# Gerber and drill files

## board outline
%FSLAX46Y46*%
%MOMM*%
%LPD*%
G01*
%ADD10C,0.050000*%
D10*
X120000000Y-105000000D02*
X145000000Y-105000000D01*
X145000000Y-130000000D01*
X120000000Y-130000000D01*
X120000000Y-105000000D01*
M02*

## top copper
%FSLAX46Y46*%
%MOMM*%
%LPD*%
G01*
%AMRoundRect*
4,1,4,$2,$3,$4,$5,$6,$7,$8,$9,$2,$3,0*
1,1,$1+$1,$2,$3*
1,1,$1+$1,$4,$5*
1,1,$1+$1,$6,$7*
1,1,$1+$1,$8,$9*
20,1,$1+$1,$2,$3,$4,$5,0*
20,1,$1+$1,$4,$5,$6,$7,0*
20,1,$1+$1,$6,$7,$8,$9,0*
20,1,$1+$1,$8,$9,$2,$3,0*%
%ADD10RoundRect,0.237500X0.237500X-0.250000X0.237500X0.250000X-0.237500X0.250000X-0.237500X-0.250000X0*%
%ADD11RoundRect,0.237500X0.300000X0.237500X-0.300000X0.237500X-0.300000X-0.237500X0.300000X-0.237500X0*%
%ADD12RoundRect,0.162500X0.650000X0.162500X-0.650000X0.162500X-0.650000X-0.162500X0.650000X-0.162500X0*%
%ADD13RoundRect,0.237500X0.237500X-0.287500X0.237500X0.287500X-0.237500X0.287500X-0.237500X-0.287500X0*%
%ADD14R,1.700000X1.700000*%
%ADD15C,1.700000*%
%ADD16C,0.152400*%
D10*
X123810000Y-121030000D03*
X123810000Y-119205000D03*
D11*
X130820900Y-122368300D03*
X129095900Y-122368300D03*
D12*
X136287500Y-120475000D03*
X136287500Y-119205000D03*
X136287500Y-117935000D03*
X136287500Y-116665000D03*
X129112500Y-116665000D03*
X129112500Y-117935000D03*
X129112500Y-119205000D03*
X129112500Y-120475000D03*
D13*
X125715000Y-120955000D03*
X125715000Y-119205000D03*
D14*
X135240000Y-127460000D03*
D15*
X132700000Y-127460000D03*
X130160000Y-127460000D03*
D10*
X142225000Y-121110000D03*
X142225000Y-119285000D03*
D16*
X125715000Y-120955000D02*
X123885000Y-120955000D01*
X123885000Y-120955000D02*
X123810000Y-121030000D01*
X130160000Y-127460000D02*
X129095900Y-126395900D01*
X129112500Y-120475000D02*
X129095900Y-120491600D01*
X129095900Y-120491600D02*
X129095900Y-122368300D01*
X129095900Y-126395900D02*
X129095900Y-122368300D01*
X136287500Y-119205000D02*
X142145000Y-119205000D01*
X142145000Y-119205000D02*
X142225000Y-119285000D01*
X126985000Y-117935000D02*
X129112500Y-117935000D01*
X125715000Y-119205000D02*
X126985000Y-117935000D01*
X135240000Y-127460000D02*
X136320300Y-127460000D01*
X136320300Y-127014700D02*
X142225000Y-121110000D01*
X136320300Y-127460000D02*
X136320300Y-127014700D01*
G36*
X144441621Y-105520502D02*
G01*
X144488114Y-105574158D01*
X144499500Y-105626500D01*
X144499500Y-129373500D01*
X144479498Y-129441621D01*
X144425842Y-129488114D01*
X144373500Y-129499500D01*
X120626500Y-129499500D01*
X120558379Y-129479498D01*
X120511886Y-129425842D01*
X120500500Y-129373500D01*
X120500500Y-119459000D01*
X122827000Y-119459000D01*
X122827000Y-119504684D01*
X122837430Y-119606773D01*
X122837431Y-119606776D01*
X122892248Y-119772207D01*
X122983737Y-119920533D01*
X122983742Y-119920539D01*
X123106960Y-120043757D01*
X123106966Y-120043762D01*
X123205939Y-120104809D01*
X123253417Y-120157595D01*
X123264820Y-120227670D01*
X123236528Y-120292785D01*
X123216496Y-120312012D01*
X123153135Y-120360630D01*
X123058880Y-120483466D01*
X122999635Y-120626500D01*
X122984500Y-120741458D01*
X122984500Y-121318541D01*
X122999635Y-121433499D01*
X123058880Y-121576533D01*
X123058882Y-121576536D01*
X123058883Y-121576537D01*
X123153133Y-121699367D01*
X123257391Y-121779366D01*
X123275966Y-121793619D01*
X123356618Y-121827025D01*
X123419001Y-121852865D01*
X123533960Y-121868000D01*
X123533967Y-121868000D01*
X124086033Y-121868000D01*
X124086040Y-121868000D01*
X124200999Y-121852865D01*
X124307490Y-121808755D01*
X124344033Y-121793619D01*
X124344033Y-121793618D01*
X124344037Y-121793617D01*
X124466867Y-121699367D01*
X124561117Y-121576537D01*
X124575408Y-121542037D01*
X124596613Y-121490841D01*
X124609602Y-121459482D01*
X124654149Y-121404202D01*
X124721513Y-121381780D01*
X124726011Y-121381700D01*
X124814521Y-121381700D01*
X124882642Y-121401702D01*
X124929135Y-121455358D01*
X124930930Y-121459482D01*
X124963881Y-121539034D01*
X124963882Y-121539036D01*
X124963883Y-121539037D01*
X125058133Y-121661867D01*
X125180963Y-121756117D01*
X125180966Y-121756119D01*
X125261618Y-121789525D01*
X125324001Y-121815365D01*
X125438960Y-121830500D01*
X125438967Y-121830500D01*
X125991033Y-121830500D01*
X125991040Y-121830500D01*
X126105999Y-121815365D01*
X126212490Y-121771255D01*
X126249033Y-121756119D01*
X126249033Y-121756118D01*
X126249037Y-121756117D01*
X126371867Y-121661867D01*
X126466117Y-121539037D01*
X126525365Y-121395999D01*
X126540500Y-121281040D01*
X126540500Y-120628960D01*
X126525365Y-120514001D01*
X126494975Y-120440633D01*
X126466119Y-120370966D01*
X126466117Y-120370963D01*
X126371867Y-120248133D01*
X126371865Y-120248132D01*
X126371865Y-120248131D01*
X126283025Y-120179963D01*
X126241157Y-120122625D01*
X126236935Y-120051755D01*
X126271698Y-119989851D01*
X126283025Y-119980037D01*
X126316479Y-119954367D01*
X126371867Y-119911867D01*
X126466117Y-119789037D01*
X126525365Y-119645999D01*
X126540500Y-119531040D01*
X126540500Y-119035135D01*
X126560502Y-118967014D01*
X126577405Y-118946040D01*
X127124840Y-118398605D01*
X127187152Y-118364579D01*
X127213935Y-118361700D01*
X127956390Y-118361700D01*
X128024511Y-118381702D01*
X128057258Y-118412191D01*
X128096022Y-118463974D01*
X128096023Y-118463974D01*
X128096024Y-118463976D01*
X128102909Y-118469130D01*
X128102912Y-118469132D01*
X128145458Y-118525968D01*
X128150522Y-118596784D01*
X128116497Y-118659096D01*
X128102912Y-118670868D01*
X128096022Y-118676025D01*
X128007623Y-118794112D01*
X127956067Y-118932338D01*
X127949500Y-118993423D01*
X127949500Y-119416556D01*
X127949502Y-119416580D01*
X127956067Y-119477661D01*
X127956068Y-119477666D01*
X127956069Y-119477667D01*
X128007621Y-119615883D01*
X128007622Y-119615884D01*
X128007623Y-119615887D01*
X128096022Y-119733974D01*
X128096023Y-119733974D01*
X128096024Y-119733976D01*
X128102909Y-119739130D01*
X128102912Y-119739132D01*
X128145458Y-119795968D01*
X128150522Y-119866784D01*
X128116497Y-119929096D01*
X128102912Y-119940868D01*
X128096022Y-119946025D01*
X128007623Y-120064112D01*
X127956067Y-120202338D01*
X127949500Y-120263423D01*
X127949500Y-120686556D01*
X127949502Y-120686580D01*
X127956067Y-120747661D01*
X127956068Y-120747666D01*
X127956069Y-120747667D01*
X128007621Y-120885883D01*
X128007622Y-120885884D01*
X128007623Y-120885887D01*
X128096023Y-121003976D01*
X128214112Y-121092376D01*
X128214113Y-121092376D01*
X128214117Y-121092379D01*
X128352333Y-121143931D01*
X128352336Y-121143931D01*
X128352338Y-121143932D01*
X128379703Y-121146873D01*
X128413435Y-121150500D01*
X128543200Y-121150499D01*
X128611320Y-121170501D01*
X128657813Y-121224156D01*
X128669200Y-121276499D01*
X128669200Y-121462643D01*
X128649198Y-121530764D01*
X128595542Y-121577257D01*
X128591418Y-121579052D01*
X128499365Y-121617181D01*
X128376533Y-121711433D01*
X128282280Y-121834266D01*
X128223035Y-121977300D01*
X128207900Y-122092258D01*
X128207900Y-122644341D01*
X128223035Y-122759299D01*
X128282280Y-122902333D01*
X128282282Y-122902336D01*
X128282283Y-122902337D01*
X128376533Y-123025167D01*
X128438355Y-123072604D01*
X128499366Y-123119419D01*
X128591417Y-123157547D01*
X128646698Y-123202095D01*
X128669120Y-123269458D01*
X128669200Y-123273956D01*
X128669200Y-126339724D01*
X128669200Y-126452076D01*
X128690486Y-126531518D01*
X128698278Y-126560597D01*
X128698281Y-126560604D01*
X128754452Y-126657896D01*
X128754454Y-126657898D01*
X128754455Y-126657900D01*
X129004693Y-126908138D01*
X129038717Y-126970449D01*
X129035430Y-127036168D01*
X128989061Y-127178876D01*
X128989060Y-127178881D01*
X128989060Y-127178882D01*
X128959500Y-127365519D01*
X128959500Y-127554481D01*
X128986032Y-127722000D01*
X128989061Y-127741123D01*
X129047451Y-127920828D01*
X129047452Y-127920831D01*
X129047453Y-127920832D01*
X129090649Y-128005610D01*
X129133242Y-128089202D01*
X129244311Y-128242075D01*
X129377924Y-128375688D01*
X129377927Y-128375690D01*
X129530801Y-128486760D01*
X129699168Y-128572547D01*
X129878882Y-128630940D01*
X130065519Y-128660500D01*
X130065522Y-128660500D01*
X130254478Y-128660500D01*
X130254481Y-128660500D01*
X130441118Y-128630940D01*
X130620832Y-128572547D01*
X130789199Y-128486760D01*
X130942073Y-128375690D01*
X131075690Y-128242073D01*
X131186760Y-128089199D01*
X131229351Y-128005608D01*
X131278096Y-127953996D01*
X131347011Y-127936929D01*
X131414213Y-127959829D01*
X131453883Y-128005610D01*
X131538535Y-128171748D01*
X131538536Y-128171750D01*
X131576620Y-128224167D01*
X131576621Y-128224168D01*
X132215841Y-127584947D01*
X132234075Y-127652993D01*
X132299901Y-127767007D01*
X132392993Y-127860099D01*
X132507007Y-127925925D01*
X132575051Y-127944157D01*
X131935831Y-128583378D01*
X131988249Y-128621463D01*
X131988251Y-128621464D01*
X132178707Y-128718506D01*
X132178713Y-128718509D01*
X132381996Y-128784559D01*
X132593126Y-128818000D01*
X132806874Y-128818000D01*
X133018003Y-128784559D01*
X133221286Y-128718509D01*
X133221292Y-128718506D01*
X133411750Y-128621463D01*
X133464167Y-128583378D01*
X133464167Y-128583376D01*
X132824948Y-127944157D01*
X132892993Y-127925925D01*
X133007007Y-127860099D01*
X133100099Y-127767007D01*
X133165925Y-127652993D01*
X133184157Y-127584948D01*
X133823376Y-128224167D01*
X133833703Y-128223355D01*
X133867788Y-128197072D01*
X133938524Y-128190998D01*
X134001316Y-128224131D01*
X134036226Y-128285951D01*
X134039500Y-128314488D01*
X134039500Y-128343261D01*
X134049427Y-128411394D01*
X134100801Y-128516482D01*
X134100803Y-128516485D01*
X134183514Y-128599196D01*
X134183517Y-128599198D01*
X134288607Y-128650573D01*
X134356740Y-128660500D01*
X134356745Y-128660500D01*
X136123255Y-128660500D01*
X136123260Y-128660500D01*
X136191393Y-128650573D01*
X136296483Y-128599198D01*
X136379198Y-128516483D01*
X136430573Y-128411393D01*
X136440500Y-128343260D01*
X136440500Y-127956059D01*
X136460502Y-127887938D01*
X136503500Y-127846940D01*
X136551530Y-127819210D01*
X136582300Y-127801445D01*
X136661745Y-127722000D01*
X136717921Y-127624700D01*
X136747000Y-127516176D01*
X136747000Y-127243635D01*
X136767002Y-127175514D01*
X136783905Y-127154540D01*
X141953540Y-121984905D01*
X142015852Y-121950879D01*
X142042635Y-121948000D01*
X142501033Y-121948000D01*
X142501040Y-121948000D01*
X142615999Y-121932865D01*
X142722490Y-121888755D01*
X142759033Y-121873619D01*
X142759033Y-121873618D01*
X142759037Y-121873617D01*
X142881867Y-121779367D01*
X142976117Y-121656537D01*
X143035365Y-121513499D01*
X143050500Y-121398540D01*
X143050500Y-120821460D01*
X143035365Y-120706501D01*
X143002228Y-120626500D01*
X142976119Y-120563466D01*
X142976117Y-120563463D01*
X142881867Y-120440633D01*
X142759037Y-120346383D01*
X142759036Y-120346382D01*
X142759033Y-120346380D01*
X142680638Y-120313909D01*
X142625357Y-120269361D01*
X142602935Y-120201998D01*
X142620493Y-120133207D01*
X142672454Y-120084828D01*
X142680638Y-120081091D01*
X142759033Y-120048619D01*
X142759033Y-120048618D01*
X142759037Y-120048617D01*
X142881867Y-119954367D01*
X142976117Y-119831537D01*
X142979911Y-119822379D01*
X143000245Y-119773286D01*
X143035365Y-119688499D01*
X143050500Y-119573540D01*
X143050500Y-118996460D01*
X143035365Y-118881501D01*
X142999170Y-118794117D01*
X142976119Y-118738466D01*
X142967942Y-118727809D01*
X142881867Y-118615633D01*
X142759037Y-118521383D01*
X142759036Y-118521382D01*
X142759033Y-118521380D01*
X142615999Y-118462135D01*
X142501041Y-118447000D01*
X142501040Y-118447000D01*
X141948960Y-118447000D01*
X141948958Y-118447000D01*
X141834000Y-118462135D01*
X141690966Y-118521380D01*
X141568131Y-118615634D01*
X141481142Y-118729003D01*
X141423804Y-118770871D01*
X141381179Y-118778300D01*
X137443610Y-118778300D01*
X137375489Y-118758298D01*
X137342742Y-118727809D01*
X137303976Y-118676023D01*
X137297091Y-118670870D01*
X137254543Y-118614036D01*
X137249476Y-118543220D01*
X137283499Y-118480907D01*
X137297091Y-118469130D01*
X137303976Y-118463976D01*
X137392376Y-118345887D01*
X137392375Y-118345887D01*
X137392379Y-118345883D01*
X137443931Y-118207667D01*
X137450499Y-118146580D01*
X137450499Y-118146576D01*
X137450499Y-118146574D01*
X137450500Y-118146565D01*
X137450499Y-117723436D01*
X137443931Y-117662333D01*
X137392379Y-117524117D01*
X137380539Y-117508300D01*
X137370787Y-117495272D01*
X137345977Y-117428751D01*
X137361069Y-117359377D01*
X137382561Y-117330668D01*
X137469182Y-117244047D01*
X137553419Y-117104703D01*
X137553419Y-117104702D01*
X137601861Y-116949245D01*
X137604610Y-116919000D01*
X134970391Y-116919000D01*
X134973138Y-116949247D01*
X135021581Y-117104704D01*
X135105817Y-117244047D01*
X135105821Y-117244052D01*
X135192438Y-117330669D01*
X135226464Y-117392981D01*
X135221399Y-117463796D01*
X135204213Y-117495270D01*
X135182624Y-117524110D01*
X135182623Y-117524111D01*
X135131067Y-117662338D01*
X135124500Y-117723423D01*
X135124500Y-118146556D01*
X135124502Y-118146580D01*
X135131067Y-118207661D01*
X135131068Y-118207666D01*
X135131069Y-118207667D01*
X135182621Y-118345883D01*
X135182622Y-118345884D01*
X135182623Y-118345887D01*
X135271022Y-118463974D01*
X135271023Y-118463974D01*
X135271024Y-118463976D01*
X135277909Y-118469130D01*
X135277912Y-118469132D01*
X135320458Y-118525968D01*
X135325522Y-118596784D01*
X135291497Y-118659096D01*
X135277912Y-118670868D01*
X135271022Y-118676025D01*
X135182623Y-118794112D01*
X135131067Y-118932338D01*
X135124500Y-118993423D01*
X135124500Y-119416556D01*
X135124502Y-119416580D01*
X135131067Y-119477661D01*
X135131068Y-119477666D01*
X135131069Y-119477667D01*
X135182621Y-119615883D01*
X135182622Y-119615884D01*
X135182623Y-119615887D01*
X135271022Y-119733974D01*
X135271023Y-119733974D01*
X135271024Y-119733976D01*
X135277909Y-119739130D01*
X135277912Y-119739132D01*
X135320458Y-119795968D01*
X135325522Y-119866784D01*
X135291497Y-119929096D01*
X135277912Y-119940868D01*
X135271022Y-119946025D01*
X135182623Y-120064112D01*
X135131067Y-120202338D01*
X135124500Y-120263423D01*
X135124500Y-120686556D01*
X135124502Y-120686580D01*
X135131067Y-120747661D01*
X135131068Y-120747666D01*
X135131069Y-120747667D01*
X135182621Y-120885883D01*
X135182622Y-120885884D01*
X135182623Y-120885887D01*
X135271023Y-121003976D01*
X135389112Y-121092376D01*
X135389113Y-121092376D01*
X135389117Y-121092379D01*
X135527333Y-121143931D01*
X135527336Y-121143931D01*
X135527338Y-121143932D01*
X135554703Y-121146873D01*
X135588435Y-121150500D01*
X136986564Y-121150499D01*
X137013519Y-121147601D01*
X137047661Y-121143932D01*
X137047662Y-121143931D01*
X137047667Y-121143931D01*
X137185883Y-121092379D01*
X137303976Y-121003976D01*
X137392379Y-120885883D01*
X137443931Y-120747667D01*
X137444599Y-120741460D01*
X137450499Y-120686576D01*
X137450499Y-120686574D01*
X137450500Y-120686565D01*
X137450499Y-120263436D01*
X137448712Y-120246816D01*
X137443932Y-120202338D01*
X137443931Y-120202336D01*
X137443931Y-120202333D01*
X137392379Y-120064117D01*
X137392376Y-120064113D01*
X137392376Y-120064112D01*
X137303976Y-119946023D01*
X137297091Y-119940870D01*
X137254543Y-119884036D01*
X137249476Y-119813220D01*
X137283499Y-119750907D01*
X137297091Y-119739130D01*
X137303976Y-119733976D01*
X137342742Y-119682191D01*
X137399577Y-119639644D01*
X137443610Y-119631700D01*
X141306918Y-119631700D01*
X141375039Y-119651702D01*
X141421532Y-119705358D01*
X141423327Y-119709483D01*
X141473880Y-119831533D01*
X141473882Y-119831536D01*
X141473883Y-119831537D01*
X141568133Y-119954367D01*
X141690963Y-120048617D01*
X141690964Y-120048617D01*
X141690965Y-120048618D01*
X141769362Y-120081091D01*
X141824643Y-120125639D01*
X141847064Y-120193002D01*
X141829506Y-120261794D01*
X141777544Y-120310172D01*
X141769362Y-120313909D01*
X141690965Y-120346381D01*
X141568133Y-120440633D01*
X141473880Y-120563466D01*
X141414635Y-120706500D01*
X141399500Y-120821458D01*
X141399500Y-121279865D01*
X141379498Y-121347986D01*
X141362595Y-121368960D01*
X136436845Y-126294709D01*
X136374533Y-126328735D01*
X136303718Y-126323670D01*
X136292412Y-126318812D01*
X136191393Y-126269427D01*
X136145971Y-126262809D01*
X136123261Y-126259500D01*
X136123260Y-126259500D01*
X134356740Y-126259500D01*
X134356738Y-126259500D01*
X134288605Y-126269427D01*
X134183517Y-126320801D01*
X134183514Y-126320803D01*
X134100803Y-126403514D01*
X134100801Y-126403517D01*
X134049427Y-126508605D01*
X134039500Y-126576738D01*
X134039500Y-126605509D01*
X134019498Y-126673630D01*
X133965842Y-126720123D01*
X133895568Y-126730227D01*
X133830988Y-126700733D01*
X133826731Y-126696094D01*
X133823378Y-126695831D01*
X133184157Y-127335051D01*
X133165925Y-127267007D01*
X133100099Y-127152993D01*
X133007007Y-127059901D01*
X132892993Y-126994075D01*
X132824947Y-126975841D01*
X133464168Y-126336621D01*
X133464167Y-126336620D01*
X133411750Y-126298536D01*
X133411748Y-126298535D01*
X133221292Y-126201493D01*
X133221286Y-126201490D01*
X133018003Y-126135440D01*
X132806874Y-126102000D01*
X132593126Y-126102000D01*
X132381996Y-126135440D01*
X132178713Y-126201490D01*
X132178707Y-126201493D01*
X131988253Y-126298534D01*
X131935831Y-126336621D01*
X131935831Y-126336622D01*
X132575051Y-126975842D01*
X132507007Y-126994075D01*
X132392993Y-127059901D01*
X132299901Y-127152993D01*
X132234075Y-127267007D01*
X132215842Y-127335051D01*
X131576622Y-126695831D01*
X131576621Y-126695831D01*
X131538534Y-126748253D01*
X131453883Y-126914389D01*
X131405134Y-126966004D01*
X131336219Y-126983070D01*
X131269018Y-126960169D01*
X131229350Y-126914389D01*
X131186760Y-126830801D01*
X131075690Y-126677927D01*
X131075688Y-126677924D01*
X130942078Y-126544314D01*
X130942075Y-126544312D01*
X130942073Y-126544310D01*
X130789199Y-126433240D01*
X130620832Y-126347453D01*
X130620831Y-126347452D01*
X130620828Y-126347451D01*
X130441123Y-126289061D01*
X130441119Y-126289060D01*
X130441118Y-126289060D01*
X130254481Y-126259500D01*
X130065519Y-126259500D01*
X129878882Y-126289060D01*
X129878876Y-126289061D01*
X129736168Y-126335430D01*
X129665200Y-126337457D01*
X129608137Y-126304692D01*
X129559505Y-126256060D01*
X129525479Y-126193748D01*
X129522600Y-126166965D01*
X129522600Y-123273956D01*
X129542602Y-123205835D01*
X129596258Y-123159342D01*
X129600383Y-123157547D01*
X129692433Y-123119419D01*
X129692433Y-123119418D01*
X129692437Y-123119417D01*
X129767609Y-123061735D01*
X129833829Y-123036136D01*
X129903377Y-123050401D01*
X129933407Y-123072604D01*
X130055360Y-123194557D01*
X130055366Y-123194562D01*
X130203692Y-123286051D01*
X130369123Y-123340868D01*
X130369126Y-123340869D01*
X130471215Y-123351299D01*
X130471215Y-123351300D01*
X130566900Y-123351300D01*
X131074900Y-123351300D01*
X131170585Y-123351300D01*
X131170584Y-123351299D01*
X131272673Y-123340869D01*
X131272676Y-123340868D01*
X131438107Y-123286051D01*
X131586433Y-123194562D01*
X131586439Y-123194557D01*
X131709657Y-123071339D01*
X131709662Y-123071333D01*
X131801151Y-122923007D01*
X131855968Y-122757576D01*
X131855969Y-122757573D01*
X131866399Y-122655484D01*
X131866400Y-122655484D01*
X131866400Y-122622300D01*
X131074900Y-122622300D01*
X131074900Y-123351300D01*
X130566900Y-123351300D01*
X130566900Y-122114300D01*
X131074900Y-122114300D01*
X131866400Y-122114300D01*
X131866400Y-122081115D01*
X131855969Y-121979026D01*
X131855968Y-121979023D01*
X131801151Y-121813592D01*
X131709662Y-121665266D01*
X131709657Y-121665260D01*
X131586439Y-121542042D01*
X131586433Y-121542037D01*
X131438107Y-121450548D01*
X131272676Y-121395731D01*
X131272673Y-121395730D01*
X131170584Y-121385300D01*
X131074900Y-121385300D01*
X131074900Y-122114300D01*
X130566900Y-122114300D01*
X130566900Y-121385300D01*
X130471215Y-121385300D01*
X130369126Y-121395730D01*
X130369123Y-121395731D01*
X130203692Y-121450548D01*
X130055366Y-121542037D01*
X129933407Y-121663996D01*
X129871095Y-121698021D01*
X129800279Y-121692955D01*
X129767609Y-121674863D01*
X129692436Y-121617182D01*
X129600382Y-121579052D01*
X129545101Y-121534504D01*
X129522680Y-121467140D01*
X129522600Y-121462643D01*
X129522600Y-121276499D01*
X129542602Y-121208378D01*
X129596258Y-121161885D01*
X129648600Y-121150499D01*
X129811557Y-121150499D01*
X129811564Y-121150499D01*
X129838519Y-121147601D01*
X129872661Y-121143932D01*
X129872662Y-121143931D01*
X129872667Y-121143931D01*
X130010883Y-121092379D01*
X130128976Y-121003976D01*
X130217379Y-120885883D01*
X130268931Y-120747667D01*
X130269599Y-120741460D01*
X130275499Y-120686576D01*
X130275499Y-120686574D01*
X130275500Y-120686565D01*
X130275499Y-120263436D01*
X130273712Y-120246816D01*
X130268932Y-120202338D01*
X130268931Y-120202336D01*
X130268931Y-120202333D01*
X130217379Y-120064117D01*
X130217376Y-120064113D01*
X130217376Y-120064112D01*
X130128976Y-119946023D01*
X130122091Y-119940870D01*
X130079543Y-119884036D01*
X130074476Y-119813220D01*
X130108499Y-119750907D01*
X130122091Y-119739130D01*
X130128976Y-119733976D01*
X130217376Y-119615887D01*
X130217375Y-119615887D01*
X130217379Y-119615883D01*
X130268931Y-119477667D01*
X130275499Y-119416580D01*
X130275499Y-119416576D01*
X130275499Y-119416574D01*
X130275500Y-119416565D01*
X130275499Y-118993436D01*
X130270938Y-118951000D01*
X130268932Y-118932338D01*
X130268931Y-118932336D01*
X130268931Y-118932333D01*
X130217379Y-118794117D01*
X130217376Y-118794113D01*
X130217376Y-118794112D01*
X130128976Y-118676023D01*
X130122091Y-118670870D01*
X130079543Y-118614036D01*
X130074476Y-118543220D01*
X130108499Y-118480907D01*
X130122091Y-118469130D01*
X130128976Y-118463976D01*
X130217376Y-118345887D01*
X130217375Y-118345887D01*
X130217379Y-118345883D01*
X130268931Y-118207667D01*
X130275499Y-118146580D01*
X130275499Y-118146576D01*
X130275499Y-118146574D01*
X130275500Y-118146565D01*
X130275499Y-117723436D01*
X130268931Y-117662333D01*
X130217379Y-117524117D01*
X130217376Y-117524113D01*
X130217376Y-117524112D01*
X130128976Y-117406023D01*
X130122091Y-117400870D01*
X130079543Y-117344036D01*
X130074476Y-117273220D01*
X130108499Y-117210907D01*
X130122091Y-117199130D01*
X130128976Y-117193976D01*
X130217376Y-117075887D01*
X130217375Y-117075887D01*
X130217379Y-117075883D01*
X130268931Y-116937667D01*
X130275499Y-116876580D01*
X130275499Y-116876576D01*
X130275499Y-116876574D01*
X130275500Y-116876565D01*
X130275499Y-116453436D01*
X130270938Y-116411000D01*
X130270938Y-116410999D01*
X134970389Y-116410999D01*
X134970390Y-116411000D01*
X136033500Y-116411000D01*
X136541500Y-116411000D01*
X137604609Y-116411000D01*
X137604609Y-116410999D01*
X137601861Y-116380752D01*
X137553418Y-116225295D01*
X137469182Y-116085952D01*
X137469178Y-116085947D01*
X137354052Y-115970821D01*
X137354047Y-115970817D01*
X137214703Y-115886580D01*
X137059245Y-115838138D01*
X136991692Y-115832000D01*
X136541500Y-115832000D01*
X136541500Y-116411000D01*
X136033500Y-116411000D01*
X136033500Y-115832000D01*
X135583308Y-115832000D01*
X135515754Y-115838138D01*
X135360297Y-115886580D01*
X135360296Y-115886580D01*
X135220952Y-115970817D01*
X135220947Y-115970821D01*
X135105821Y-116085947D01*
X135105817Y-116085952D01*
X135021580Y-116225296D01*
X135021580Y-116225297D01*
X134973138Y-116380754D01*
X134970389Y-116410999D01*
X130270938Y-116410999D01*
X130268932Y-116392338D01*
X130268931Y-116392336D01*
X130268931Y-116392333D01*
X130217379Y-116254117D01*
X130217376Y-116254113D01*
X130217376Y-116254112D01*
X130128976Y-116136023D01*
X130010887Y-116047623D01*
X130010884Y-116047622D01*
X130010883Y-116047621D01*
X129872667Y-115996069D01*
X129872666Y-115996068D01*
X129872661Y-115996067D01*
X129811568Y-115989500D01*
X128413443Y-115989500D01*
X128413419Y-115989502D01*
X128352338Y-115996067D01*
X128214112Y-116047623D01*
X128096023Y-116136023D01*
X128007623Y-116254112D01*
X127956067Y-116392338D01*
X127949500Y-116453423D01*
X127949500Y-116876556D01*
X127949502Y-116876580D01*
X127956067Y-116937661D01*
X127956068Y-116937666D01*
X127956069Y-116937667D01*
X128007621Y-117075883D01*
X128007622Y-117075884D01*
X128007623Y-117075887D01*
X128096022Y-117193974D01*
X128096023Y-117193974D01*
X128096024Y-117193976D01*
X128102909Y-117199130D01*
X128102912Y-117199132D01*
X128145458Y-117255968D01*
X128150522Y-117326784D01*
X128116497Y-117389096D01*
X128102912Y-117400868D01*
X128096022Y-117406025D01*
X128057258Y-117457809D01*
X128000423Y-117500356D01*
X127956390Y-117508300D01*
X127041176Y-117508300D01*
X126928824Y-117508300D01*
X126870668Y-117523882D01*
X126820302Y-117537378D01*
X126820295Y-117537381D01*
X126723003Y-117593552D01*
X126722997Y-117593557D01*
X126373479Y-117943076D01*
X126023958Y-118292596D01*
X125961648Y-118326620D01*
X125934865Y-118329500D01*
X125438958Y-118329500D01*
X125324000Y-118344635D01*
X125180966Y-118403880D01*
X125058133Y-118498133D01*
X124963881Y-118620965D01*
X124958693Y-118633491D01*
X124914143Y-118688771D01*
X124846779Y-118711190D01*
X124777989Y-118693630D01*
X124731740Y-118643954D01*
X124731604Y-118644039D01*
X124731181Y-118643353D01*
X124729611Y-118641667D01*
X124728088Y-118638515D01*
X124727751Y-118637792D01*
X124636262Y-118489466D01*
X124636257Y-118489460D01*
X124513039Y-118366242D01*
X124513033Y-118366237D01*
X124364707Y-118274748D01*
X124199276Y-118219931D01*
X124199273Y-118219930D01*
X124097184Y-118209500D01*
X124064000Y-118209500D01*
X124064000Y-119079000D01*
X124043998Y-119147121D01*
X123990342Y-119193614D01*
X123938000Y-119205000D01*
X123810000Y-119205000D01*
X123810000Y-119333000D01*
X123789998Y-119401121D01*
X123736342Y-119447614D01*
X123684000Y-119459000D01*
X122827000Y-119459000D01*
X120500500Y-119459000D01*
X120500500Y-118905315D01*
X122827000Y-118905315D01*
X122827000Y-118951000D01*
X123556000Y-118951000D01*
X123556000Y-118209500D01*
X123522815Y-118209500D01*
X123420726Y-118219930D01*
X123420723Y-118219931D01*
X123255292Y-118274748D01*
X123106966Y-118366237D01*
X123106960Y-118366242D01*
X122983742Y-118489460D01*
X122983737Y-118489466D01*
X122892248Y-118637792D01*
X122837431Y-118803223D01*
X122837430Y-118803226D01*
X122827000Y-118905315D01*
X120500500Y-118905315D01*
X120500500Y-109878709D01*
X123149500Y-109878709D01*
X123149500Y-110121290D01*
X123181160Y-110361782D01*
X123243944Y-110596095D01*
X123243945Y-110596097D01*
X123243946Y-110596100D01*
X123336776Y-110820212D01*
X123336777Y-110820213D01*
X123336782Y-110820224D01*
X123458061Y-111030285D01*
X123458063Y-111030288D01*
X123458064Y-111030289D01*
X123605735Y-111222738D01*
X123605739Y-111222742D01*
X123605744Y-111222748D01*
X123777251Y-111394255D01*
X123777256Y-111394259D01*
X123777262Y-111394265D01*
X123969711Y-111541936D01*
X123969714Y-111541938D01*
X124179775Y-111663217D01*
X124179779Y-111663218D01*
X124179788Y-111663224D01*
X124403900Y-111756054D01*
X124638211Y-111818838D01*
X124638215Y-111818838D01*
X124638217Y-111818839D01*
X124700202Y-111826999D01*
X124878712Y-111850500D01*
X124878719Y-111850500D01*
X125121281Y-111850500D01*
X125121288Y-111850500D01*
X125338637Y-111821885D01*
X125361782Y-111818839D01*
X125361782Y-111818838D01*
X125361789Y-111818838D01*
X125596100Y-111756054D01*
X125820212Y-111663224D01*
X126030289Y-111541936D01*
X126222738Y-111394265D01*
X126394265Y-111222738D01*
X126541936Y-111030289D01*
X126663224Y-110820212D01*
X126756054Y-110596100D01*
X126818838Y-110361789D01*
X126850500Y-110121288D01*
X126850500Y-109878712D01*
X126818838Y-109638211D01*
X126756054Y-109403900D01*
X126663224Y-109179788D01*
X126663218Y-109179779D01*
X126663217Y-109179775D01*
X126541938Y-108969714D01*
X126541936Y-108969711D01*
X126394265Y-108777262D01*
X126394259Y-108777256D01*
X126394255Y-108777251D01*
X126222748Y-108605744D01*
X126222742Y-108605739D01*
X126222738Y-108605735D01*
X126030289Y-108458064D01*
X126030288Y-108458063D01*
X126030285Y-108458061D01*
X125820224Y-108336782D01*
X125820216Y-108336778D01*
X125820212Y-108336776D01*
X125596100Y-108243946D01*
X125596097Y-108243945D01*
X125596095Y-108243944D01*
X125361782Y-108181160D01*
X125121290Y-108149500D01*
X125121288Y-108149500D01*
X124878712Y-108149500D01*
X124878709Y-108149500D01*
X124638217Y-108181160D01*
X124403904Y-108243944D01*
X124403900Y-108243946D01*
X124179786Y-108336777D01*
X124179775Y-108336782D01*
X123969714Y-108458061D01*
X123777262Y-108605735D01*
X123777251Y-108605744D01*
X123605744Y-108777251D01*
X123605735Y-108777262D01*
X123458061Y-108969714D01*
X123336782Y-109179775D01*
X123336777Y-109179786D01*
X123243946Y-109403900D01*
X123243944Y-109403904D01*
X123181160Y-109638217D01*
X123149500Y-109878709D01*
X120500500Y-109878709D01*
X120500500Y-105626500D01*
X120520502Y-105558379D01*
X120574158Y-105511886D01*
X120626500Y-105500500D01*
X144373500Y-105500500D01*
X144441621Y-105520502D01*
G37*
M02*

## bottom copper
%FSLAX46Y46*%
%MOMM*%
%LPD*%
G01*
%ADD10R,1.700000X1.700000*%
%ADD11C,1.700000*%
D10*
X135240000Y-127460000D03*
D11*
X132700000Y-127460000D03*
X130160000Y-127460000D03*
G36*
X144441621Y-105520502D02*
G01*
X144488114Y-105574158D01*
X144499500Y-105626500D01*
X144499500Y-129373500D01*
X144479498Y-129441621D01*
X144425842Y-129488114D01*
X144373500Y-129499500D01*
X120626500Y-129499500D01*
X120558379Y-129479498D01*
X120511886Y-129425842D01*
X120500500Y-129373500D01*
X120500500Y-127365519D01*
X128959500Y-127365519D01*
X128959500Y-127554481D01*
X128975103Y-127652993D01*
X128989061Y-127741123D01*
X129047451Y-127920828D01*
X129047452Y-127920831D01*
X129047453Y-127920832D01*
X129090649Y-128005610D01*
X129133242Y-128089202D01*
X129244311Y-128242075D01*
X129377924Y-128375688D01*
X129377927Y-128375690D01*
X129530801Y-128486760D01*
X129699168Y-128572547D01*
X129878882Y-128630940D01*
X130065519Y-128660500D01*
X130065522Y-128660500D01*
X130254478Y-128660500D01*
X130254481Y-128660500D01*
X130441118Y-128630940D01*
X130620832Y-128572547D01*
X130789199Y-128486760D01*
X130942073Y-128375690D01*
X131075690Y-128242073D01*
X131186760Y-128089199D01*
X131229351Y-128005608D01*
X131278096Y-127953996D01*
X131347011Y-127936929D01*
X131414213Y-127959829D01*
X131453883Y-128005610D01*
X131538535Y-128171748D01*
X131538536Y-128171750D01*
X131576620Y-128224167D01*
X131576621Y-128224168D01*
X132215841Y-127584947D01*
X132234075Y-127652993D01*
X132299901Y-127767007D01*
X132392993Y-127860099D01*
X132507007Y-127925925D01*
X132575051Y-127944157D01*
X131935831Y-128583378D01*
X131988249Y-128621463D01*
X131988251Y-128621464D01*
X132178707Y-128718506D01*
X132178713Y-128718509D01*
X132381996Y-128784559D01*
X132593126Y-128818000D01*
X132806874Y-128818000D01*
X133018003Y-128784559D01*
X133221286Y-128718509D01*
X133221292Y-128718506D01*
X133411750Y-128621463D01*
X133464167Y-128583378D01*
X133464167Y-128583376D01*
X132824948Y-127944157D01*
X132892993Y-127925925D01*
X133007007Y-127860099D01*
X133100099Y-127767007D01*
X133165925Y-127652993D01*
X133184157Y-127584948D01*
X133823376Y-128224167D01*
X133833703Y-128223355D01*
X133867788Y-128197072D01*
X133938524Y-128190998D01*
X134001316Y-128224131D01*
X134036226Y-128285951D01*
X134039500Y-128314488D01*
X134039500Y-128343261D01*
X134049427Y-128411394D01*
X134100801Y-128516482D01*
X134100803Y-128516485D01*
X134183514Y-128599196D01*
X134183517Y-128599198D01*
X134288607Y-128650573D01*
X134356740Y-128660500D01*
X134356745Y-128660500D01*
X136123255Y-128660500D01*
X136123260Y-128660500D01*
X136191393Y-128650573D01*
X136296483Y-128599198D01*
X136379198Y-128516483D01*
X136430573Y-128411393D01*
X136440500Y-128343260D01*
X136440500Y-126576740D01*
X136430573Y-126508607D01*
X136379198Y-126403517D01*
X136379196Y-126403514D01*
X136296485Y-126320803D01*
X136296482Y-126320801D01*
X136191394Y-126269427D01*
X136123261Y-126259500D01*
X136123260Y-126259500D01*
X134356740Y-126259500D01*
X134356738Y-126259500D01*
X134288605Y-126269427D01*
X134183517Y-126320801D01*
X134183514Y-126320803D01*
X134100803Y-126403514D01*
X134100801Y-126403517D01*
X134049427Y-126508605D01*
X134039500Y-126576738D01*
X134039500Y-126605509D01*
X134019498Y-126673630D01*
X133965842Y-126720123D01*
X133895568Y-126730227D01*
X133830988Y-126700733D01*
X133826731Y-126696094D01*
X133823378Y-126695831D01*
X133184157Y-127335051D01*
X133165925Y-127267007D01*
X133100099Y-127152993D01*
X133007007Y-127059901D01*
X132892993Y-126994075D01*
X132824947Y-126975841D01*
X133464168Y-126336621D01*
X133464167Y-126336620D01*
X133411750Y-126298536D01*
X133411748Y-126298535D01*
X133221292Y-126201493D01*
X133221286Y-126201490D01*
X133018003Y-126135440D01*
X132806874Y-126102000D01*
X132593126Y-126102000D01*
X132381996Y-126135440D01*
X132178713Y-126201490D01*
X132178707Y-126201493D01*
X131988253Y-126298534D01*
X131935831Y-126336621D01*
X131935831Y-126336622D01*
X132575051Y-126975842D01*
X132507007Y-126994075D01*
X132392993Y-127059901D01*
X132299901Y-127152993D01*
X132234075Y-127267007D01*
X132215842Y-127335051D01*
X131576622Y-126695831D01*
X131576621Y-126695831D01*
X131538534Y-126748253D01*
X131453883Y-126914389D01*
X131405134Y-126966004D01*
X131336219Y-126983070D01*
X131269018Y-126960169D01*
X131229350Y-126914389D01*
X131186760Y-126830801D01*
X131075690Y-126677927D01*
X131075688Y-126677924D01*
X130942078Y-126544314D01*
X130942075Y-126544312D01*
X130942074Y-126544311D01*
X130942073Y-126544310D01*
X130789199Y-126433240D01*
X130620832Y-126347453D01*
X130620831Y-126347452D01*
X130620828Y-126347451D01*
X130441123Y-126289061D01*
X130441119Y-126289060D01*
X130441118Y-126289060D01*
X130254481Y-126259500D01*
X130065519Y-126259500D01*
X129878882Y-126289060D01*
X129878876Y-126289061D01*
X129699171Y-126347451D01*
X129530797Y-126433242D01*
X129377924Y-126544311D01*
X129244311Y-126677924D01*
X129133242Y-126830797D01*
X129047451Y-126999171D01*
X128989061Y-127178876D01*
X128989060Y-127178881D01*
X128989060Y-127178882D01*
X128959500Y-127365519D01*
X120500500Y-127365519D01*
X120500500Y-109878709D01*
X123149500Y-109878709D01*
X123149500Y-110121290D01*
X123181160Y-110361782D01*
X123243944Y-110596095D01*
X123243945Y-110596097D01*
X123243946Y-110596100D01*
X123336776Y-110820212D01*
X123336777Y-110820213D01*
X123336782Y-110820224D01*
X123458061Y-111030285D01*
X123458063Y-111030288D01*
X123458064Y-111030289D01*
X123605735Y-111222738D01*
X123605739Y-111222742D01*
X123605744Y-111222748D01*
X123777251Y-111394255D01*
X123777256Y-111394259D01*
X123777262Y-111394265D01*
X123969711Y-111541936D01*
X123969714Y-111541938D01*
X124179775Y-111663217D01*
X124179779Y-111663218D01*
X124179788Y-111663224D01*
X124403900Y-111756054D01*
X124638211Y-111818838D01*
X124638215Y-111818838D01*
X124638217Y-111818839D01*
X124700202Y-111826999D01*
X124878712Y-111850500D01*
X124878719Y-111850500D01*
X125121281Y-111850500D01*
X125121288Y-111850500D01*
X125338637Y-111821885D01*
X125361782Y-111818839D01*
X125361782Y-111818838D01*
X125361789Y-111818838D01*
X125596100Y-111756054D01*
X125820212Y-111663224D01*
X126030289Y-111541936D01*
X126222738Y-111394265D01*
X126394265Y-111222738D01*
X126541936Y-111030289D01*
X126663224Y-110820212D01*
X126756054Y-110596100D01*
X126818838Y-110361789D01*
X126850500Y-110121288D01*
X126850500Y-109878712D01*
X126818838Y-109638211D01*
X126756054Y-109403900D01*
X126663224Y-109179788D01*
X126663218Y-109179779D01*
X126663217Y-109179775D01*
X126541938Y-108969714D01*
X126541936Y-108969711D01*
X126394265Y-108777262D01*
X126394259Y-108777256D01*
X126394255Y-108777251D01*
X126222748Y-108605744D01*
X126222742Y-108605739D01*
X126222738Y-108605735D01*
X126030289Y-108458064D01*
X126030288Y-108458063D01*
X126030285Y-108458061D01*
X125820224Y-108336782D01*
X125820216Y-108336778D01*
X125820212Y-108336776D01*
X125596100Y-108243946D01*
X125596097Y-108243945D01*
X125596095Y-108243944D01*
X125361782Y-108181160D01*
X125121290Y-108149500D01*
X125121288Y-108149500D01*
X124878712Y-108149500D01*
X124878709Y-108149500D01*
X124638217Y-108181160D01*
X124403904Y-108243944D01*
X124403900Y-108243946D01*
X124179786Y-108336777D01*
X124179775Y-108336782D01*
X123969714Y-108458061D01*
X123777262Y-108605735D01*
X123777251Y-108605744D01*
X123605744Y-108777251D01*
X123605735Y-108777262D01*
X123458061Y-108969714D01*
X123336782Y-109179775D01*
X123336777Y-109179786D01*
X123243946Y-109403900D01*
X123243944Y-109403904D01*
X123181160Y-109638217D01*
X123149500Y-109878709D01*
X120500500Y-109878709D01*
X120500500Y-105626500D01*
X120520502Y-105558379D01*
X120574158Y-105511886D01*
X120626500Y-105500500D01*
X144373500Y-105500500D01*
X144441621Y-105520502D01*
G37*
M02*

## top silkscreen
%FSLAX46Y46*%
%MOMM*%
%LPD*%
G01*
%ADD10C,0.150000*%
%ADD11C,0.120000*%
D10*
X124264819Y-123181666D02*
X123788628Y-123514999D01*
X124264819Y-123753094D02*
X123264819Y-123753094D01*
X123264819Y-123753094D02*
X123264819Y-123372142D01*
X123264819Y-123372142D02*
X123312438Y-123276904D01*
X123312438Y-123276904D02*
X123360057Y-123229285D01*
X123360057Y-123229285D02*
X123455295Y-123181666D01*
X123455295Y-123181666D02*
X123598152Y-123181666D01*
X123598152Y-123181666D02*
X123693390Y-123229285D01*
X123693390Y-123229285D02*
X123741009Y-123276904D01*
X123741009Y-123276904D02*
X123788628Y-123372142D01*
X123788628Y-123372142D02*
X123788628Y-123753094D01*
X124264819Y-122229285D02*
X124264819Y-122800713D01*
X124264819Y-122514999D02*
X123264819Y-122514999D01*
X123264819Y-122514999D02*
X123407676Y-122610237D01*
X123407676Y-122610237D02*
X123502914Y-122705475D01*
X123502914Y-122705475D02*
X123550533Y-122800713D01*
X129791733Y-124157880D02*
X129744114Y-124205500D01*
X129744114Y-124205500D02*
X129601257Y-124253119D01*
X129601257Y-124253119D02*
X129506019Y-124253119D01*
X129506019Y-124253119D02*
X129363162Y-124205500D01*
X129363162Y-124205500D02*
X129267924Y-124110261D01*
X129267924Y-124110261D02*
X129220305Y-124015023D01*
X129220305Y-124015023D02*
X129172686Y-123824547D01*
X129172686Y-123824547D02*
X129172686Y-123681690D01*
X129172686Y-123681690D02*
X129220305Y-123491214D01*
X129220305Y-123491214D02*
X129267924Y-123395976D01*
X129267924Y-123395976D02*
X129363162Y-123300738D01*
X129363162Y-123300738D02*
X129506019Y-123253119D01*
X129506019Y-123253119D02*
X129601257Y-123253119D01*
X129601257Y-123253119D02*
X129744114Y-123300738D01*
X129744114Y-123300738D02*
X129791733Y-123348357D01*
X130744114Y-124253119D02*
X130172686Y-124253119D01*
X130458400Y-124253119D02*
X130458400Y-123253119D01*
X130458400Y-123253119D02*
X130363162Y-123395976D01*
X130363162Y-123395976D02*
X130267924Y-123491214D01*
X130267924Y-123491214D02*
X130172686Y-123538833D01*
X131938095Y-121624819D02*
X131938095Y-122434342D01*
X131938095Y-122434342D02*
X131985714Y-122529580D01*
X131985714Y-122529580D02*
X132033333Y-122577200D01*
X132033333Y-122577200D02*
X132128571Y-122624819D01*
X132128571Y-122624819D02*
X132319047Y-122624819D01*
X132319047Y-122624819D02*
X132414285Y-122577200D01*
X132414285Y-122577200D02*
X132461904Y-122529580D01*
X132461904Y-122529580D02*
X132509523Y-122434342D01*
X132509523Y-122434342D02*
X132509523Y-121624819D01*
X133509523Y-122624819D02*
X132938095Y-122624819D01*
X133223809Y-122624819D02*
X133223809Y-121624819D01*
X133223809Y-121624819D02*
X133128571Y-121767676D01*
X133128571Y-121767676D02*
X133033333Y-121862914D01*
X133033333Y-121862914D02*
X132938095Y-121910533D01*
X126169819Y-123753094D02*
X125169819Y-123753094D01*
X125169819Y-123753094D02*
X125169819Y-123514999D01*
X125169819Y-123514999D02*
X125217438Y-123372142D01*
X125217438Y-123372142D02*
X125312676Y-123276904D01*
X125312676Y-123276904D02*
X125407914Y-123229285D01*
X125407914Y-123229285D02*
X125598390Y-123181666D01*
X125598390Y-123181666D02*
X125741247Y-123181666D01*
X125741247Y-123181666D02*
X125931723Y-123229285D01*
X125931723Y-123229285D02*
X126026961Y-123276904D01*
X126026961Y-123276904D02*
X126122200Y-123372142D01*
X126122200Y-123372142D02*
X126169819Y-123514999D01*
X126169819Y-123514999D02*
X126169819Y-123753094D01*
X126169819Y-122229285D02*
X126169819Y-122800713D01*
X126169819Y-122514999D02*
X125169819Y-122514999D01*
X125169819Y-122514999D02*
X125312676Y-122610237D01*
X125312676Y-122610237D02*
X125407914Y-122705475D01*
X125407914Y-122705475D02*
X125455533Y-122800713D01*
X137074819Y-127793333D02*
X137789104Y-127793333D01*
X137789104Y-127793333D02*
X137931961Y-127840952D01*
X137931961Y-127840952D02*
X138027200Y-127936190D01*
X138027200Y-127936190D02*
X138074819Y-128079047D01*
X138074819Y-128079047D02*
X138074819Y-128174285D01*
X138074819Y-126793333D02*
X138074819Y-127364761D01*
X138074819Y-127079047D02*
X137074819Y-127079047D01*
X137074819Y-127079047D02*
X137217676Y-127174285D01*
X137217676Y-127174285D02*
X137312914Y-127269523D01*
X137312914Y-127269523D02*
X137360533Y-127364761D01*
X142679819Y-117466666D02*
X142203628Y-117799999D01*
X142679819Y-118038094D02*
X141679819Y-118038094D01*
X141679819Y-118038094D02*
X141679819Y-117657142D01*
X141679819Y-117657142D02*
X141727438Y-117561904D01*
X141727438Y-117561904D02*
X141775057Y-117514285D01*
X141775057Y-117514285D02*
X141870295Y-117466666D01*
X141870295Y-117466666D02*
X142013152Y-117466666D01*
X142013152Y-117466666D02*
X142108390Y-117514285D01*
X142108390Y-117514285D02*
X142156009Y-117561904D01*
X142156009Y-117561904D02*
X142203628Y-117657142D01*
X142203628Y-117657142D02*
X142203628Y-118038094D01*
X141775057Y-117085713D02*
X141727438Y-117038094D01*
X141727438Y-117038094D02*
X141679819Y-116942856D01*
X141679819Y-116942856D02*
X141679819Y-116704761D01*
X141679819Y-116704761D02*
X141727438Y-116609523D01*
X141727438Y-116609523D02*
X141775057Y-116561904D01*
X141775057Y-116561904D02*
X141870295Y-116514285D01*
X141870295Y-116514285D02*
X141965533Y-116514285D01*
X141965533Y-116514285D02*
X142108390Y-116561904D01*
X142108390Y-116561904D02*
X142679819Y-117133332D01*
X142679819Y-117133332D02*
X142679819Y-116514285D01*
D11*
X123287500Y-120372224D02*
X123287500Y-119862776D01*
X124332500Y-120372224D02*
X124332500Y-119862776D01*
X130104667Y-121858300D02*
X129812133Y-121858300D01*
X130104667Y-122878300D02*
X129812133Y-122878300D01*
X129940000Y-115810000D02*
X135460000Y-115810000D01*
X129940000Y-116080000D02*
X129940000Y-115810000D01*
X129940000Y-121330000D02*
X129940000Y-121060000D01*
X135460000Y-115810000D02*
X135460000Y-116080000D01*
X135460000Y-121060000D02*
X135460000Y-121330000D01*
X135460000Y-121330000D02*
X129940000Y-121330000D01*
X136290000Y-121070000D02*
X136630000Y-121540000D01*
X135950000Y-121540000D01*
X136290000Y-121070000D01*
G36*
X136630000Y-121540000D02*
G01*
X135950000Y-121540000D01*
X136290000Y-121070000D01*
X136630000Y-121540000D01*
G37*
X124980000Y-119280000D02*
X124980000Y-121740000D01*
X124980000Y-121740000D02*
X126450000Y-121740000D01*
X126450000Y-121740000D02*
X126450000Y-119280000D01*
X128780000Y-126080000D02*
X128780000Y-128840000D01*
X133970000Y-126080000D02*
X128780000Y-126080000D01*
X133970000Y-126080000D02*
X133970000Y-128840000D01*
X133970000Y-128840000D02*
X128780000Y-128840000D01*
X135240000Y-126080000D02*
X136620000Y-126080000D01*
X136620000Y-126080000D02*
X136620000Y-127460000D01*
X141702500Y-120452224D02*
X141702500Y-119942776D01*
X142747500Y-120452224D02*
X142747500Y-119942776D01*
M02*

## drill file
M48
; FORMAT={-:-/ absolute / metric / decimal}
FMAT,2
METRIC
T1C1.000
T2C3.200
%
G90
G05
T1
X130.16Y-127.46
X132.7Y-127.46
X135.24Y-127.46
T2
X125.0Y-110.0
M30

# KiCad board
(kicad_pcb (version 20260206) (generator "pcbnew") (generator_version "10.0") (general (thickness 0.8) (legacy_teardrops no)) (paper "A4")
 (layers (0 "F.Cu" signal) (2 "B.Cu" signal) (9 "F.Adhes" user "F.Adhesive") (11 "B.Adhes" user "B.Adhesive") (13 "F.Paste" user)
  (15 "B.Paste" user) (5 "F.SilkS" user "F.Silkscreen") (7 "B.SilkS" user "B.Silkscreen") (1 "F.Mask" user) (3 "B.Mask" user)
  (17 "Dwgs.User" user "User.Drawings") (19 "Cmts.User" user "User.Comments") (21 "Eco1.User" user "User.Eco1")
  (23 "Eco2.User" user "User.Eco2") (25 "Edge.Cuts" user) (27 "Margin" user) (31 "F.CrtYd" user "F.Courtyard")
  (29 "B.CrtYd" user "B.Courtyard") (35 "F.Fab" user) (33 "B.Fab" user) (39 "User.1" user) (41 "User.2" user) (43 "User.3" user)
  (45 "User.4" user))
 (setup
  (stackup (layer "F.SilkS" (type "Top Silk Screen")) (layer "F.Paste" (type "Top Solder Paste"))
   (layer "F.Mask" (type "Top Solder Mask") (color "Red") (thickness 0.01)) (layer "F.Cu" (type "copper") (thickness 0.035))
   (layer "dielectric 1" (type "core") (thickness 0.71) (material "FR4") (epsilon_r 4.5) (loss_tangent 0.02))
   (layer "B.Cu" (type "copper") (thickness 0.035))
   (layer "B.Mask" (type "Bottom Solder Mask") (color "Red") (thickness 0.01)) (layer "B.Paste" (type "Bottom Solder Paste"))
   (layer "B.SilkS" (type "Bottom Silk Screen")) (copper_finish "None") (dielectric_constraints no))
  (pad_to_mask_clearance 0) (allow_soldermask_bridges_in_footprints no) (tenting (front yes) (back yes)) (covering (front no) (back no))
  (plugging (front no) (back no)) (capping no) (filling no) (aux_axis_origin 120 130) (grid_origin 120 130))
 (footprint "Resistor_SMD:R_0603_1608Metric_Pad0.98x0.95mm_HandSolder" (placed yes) (layer "F.Cu") (at 123.81 120.1175 90)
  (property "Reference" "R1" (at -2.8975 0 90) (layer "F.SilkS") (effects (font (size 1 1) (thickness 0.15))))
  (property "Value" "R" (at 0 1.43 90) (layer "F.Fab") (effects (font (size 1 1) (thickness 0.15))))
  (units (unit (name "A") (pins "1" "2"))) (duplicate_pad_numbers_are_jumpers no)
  (fp_line (start -0.254724 -0.5225) (end 0.254724 -0.5225) (stroke (width 0.12) (type solid)) (layer "F.SilkS"))
  (fp_line (start -0.254724 0.5225) (end 0.254724 0.5225) (stroke (width 0.12) (type solid)) (layer "F.SilkS"))
  (pad "1" smd roundrect (at -0.9125 0 90) (size 0.975 0.95) (layers "F.Cu" "F.Mask" "F.Paste") (roundrect_rratio 0.25) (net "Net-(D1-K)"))
  (pad "2" smd roundrect (at 0.9125 0 90) (size 0.975 0.95) (layers "F.Cu" "F.Mask" "F.Paste") (roundrect_rratio 0.25) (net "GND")))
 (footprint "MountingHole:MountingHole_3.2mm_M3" (layer "F.Cu") (at 125 110)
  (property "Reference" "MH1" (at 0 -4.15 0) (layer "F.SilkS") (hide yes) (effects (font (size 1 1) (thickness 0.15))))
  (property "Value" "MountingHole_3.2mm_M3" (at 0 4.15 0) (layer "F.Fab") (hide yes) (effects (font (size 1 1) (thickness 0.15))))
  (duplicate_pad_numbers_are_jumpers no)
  (pad "" np_thru_hole circle (at 0 0) (size 3.2 3.2) (drill 3.2) (layers "*.Cu" "*.Mask")))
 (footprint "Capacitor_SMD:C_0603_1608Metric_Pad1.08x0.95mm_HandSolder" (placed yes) (layer "F.Cu") (at 129.9584 122.3683 180)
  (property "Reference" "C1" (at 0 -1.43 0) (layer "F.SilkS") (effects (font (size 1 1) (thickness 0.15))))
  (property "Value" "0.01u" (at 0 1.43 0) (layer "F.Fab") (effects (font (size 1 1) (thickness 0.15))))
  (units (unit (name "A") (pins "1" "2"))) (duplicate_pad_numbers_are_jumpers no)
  (fp_line (start -0.146267 0.51) (end 0.146267 0.51) (stroke (width 0.12) (type solid)) (layer "F.SilkS"))
  (fp_line (start -0.146267 -0.51) (end 0.146267 -0.51) (stroke (width 0.12) (type solid)) (layer "F.SilkS"))
  (pad "1" smd roundrect (at -0.8625 0 180) (size 1.075 0.95) (layers "F.Cu" "F.Mask" "F.Paste") (roundrect_rratio 0.25) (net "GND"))
  (pad "2" smd roundrect (at 0.8625 0 180) (size 1.075 0.95) (layers "F.Cu" "F.Mask" "F.Paste") (roundrect_rratio 0.25) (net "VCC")))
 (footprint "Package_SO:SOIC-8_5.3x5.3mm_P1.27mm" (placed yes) (layer "F.Cu") (at 132.7 118.57 180)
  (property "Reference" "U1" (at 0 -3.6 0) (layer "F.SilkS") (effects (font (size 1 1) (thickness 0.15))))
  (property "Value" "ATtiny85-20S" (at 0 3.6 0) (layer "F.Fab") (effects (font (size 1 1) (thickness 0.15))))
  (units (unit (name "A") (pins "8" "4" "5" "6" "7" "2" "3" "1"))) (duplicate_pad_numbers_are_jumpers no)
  (fp_line (start 2.76 2.76) (end -2.76 2.76) (stroke (width 0.12) (type solid)) (layer "F.SilkS"))
  (fp_line (start 2.76 2.49) (end 2.76 2.76) (stroke (width 0.12) (type solid)) (layer "F.SilkS"))
  (fp_line (start 2.76 -2.76) (end 2.76 -2.49) (stroke (width 0.12) (type solid)) (layer "F.SilkS"))
  (fp_line (start -2.76 2.76) (end -2.76 2.49) (stroke (width 0.12) (type solid)) (layer "F.SilkS"))
  (fp_line (start -2.76 -2.49) (end -2.76 -2.76) (stroke (width 0.12) (type solid)) (layer "F.SilkS"))
  (fp_line (start -2.76 -2.76) (end 2.76 -2.76) (stroke (width 0.12) (type solid)) (layer "F.SilkS"))
  (fp_poly (pts (xy -3.59 -2.5) (xy -3.93 -2.97) (xy -3.25 -2.97)) (stroke (width 0.12) (type solid)) (fill yes) (layer "F.SilkS"))
  (pad "1" smd roundrect (at -3.5875 -1.905 180) (size 1.625 0.65) (layers "F.Cu" "F.Mask" "F.Paste") (roundrect_rratio 0.25)
   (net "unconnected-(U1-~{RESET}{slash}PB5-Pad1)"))
  (pad "2" smd roundrect (at -3.5875 -0.635 180) (size 1.625 0.65) (layers "F.Cu" "F.Mask" "F.Paste") (roundrect_rratio 0.25) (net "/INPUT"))
  (pad "3" smd roundrect (at -3.5875 0.635 180) (size 1.625 0.65) (layers "F.Cu" "F.Mask" "F.Paste") (roundrect_rratio 0.25)
   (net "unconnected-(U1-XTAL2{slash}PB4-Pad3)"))
  (pad "4" smd roundrect (at -3.5875 1.905 180) (size 1.625 0.65) (layers "F.Cu" "F.Mask" "F.Paste") (roundrect_rratio 0.25) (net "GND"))
  (pad "5" smd roundrect (at 3.5875 1.905 180) (size 1.625 0.65) (layers "F.Cu" "F.Mask" "F.Paste") (roundrect_rratio 0.25)
   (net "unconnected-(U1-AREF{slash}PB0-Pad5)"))
  (pad "6" smd roundrect (at 3.5875 0.635 180) (size 1.625 0.65) (layers "F.Cu" "F.Mask" "F.Paste") (roundrect_rratio 0.25)
   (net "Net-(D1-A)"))
  (pad "7" smd roundrect (at 3.5875 -0.635 180) (size 1.625 0.65) (layers "F.Cu" "F.Mask" "F.Paste") (roundrect_rratio 0.25)
   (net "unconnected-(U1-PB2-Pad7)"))
  (pad "8" smd roundrect (at 3.5875 -1.905 180) (size 1.625 0.65) (layers "F.Cu" "F.Mask" "F.Paste") (roundrect_rratio 0.25) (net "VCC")))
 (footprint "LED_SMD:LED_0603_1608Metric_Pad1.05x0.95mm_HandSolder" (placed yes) (layer "F.Cu") (at 125.715 120.08 90)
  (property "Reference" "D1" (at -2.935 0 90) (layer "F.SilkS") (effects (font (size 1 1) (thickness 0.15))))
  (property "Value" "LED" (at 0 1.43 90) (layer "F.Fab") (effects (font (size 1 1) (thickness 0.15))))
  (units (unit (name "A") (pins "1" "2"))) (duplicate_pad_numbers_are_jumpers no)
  (fp_line (start 0.8 -0.735) (end -1.66 -0.735) (stroke (width 0.12) (type solid)) (layer "F.SilkS"))
  (fp_line (start -1.66 -0.735) (end -1.66 0.735) (stroke (width 0.12) (type solid)) (layer "F.SilkS"))
  (fp_line (start -1.66 0.735) (end 0.8 0.735) (stroke (width 0.12) (type solid)) (layer "F.SilkS"))
  (pad "1" smd roundrect (at -0.875 0 90) (size 1.05 0.95) (layers "F.Cu" "F.Mask" "F.Paste") (roundrect_rratio 0.25) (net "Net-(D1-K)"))
  (pad "2" smd roundrect (at 0.875 0 90) (size 1.05 0.95) (layers "F.Cu" "F.Mask" "F.Paste") (roundrect_rratio 0.25) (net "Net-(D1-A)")))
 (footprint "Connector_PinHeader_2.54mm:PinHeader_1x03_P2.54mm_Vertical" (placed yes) (layer "F.Cu") (at 135.24 127.46 -90)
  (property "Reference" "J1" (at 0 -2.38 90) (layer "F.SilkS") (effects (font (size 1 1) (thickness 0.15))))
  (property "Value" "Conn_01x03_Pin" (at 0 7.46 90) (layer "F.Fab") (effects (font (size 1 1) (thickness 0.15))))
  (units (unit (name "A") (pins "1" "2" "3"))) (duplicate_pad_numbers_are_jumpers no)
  (fp_line (start -1.38 6.46) (end 1.38 6.46) (stroke (width 0.12) (type solid)) (layer "F.SilkS"))
  (fp_line (start -1.38 1.27) (end -1.38 6.46) (stroke (width 0.12) (type solid)) (layer "F.SilkS"))
  (fp_line (start -1.38 1.27) (end 1.38 1.27) (stroke (width 0.12) (type solid)) (layer "F.SilkS"))
  (fp_line (start 1.38 1.27) (end 1.38 6.46) (stroke (width 0.12) (type solid)) (layer "F.SilkS"))
  (fp_line (start -1.38 0) (end -1.38 -1.38) (stroke (width 0.12) (type solid)) (layer "F.SilkS"))
  (fp_line (start -1.38 -1.38) (end 0 -1.38) (stroke (width 0.12) (type solid)) (layer "F.SilkS"))
  (pad "1" thru_hole rect (at 0 0 270) (size 1.7 1.7) (drill 1) (layers "*.Cu" "*.Mask") (remove_unused_layers no) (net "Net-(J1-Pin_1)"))
  (pad "2" thru_hole circle (at 0 2.54 270) (size 1.7 1.7) (drill 1) (layers "*.Cu" "*.Mask") (remove_unused_layers no) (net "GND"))
  (pad "3" thru_hole circle (at 0 5.08 270) (size 1.7 1.7) (drill 1) (layers "*.Cu" "*.Mask") (remove_unused_layers no) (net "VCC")))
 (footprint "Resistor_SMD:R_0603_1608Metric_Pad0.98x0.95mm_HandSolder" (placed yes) (layer "F.Cu") (at 142.225 120.1975 90)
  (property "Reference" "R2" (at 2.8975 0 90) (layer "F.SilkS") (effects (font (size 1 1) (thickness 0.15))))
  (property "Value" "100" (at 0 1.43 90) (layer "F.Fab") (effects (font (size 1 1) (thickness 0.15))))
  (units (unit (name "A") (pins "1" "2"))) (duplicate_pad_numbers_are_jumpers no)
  (fp_line (start -0.254724 -0.5225) (end 0.254724 -0.5225) (stroke (width 0.12) (type solid)) (layer "F.SilkS"))
  (fp_line (start -0.254724 0.5225) (end 0.254724 0.5225) (stroke (width 0.12) (type solid)) (layer "F.SilkS"))
  (pad "1" smd roundrect (at -0.9125 0 90) (size 0.975 0.95) (layers "F.Cu" "F.Mask" "F.Paste") (roundrect_rratio 0.25)
   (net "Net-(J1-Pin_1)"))
  (pad "2" smd roundrect (at 0.9125 0 90) (size 0.975 0.95) (layers "F.Cu" "F.Mask" "F.Paste") (roundrect_rratio 0.25) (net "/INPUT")))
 (gr_rect (start 120 105) (end 145 130) (stroke (width 0.05) (type solid)) (fill no) (layer "Edge.Cuts"))
 (segment (start 125.715 120.955) (end 123.885 120.955) (width 0.1524) (layer "F.Cu") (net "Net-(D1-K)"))
 (segment (start 123.885 120.955) (end 123.81 121.03) (width 0.1524) (layer "F.Cu") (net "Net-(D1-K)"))
 (segment (start 130.16 127.46) (end 129.0959 126.3959) (width 0.1524) (layer "F.Cu") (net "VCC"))
 (segment (start 129.1125 120.475) (end 129.0959 120.4916) (width 0.1524) (layer "F.Cu") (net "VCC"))
 (segment (start 129.0959 120.4916) (end 129.0959 122.3683) (width 0.1524) (layer "F.Cu") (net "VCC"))
 (segment (start 129.0959 126.3959) (end 129.0959 122.3683) (width 0.1524) (layer "F.Cu") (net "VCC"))
 (segment (start 136.2875 119.205) (end 142.145 119.205) (width 0.1524) (layer "F.Cu") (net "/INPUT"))
 (segment (start 142.145 119.205) (end 142.225 119.285) (width 0.1524) (layer "F.Cu") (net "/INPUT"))
 (segment (start 126.985 117.935) (end 129.1125 117.935) (width 0.1524) (layer "F.Cu") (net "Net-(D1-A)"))
 (segment (start 125.715 119.205) (end 126.985 117.935) (width 0.1524) (layer "F.Cu") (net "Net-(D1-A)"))
 (segment (start 135.24 127.46) (end 136.3203 127.46) (width 0.1524) (layer "F.Cu") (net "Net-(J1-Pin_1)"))
 (segment (start 136.3203 127.0147) (end 142.225 121.11) (width 0.1524) (layer "F.Cu") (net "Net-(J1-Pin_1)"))
 (segment (start 136.3203 127.46) (end 136.3203 127.0147) (width 0.1524) (layer "F.Cu") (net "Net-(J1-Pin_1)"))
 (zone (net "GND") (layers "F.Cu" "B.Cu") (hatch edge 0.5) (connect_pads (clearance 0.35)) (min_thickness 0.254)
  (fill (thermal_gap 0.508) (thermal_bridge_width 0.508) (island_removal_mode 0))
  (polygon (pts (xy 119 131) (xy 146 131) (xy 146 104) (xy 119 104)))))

